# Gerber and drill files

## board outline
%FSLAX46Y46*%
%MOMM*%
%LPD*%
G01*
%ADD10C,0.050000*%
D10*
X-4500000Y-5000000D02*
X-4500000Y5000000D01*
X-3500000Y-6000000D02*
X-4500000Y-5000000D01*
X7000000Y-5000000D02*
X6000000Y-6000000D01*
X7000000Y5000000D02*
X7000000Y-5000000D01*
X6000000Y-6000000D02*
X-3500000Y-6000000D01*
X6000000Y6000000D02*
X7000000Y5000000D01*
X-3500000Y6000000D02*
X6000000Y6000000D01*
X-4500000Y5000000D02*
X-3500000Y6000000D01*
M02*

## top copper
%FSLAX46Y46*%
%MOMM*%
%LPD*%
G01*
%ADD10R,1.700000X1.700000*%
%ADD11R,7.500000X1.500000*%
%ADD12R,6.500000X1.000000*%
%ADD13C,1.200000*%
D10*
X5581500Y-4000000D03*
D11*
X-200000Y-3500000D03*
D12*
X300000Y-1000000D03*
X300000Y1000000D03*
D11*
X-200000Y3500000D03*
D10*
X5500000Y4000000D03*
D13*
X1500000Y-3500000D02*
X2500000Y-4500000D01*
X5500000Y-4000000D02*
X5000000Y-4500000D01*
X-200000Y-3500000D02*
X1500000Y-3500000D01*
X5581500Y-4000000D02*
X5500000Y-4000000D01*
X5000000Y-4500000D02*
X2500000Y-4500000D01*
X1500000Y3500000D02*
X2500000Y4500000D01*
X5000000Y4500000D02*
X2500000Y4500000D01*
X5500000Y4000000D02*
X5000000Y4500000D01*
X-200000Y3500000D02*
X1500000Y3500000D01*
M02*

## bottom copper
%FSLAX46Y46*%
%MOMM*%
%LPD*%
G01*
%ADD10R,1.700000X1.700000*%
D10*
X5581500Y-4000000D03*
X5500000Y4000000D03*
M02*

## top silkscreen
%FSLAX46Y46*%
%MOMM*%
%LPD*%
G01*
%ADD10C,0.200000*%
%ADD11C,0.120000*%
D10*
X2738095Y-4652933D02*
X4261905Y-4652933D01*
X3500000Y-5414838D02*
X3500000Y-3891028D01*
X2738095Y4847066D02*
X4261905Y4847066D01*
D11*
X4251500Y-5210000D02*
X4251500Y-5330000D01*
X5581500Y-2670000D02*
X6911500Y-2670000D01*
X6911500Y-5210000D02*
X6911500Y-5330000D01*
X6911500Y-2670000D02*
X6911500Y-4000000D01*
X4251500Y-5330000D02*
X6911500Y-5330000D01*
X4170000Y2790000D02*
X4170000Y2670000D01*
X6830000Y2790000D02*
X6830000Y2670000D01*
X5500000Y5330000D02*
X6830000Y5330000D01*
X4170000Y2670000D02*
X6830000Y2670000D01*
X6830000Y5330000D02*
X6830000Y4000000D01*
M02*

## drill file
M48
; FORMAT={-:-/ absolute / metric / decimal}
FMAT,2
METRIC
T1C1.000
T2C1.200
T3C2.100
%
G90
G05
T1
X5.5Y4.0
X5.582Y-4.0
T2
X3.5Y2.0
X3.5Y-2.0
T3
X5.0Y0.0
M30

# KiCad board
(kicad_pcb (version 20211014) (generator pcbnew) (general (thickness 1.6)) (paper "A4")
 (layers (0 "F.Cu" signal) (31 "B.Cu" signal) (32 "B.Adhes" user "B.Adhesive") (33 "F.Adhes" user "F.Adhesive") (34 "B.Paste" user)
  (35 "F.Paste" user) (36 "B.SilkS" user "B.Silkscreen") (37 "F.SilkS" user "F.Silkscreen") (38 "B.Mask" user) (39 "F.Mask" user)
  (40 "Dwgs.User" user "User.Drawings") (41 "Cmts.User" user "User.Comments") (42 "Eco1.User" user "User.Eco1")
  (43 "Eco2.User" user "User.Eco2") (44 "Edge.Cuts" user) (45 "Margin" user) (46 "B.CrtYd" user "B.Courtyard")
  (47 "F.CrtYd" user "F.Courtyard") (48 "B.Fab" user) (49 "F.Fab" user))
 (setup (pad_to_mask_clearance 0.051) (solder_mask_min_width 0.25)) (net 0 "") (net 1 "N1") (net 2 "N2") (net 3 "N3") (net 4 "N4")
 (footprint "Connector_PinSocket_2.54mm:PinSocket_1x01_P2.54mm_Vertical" (layer "F.Cu") (at 5.5815 4)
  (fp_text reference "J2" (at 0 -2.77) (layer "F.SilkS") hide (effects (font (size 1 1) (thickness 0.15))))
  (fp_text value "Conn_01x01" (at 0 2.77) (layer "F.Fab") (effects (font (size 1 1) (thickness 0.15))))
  (fp_line (start -1.33 1.21) (end -1.33 1.33) (layer "F.SilkS") (width 0.12))
  (fp_line (start 0 -1.33) (end 1.33 -1.33) (layer "F.SilkS") (width 0.12))
  (fp_line (start 1.33 1.21) (end 1.33 1.33) (layer "F.SilkS") (width 0.12))
  (fp_line (start 1.33 -1.33) (end 1.33 0) (layer "F.SilkS") (width 0.12))
  (fp_line (start -1.33 1.33) (end 1.33 1.33) (layer "F.SilkS") (width 0.12))
  (pad "1" thru_hole rect locked (at 0 0) (size 1.7 1.7) (drill 1) (layers *.Cu *.Mask) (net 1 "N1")))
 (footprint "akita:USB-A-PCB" (layer "F.Cu") (at 0 0)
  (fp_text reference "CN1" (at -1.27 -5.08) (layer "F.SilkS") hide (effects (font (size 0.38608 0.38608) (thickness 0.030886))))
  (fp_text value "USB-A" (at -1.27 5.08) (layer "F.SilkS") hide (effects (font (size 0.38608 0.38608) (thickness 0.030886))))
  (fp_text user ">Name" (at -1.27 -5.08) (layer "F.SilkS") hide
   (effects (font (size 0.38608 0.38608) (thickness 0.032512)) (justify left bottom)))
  (pad "1" smd rect locked (at -0.2 3.5) (size 7.5 1.5) (layers "F.Cu" "F.Paste" "F.Mask") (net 1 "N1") (solder_mask_margin 0.1016))
  (pad "2" smd rect locked (at 0.3 1) (size 6.5 1) (layers "F.Cu" "F.Paste" "F.Mask") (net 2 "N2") (solder_mask_margin 0.1016))
  (pad "3" smd rect locked (at 0.3 -1) (size 6.5 1) (layers "F.Cu" "F.Paste" "F.Mask") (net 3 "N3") (solder_mask_margin 0.1016))
  (pad "4" smd rect locked (at -0.2 -3.5) (size 7.5 1.5) (layers "F.Cu" "F.Paste" "F.Mask") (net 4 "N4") (solder_mask_margin 0.1016)))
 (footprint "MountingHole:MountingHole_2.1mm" (layer "F.Cu") (at 5 0)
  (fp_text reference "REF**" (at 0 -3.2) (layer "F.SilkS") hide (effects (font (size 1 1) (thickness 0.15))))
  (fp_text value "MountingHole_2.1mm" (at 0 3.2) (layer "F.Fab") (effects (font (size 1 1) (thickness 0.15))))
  (pad "" np_thru_hole circle locked (at 0 0) (size 2.1 2.1) (drill 2.1) (layers *.Cu *.Mask)))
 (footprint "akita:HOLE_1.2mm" (layer "F.Cu") (at 3.5 -2)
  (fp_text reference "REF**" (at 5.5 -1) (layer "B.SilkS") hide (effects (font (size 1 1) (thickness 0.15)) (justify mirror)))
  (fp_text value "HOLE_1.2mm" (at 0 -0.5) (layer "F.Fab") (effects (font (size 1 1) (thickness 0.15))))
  (pad "" np_thru_hole circle locked (at 0 0) (size 1.2 1.2) (drill 1.2) (layers *.Cu *.Mask) (solder_mask_margin 0.1016)))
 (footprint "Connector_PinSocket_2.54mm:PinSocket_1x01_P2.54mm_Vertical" (layer "F.Cu") (at 5.5 -4)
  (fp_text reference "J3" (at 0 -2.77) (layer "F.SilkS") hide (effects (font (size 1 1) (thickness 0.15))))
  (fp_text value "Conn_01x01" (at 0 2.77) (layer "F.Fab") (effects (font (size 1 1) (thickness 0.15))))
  (fp_line (start -1.33 1.21) (end -1.33 1.33) (layer "F.SilkS") (width 0.12))
  (fp_line (start 1.33 1.21) (end 1.33 1.33) (layer "F.SilkS") (width 0.12))
  (fp_line (start 0 -1.33) (end 1.33 -1.33) (layer "F.SilkS") (width 0.12))
  (fp_line (start -1.33 1.33) (end 1.33 1.33) (layer "F.SilkS") (width 0.12))
  (fp_line (start 1.33 -1.33) (end 1.33 0) (layer "F.SilkS") (width 0.12))
  (pad "1" thru_hole rect locked (at 0 0) (size 1.7 1.7) (drill 1) (layers *.Cu *.Mask) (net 4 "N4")))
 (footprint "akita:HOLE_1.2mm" (layer "B.Cu") (at 3.5 2)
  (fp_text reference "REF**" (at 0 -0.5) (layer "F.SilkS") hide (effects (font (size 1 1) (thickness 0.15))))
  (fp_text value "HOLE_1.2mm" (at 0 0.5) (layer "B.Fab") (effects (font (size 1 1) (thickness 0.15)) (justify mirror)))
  (pad "" np_thru_hole circle locked (at 0 0) (size 1.2 1.2) (drill 1.2) (layers *.Cu *.Mask) (solder_mask_margin 0.1016)))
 (gr_line (start -4.5 5) (end -4.5 -5) (layer "Edge.Cuts") (width 0.05))
 (gr_line (start -3.5 6) (end -4.5 5) (layer "Edge.Cuts") (width 0.05))
 (gr_line (start 7 5) (end 6 6) (layer "Edge.Cuts") (width 0.05))
 (gr_line (start 7 -5) (end 7 5) (layer "Edge.Cuts") (width 0.05))
 (gr_line (start 6 6) (end -3.5 6) (layer "Edge.Cuts") (width 0.05))
 (gr_line (start 6 -6) (end 7 -5) (layer "Edge.Cuts") (width 0.05))
 (gr_line (start -3.5 -6) (end 6 -6) (layer "Edge.Cuts") (width 0.05))
 (gr_line (start -4.5 -5) (end -3.5 -6) (layer "Edge.Cuts") (width 0.05))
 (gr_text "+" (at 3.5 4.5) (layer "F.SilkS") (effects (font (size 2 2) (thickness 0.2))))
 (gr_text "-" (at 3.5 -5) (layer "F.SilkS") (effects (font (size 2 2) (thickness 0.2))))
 (segment (start 1.5 3.5) (end 2.5 4.5) (width 1.2) (layer "F.Cu") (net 1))
 (segment (start 5.5 4) (end 5 4.5) (width 1.2) (layer "F.Cu") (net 1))
 (segment (start -0.2 3.5) (end 1.5 3.5) (width 1.2) (layer "F.Cu") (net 1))
 (segment (start 5.5815 4) (end 5.5 4) (width 1.2) (layer "F.Cu") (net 1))
 (segment (start 5 4.5) (end 2.5 4.5) (width 1.2) (layer "F.Cu") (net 1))
 (segment (start 1.5 -3.5) (end 2.5 -4.5) (width 1.2) (layer "F.Cu") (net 4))
 (segment (start 5 -4.5) (end 2.5 -4.5) (width 1.2) (layer "F.Cu") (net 4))
 (segment (start 5.5 -4) (end 5 -4.5) (width 1.2) (layer "F.Cu") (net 4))
 (segment (start -0.2 -3.5) (end 1.5 -3.5) (width 1.2) (layer "F.Cu") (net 4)))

